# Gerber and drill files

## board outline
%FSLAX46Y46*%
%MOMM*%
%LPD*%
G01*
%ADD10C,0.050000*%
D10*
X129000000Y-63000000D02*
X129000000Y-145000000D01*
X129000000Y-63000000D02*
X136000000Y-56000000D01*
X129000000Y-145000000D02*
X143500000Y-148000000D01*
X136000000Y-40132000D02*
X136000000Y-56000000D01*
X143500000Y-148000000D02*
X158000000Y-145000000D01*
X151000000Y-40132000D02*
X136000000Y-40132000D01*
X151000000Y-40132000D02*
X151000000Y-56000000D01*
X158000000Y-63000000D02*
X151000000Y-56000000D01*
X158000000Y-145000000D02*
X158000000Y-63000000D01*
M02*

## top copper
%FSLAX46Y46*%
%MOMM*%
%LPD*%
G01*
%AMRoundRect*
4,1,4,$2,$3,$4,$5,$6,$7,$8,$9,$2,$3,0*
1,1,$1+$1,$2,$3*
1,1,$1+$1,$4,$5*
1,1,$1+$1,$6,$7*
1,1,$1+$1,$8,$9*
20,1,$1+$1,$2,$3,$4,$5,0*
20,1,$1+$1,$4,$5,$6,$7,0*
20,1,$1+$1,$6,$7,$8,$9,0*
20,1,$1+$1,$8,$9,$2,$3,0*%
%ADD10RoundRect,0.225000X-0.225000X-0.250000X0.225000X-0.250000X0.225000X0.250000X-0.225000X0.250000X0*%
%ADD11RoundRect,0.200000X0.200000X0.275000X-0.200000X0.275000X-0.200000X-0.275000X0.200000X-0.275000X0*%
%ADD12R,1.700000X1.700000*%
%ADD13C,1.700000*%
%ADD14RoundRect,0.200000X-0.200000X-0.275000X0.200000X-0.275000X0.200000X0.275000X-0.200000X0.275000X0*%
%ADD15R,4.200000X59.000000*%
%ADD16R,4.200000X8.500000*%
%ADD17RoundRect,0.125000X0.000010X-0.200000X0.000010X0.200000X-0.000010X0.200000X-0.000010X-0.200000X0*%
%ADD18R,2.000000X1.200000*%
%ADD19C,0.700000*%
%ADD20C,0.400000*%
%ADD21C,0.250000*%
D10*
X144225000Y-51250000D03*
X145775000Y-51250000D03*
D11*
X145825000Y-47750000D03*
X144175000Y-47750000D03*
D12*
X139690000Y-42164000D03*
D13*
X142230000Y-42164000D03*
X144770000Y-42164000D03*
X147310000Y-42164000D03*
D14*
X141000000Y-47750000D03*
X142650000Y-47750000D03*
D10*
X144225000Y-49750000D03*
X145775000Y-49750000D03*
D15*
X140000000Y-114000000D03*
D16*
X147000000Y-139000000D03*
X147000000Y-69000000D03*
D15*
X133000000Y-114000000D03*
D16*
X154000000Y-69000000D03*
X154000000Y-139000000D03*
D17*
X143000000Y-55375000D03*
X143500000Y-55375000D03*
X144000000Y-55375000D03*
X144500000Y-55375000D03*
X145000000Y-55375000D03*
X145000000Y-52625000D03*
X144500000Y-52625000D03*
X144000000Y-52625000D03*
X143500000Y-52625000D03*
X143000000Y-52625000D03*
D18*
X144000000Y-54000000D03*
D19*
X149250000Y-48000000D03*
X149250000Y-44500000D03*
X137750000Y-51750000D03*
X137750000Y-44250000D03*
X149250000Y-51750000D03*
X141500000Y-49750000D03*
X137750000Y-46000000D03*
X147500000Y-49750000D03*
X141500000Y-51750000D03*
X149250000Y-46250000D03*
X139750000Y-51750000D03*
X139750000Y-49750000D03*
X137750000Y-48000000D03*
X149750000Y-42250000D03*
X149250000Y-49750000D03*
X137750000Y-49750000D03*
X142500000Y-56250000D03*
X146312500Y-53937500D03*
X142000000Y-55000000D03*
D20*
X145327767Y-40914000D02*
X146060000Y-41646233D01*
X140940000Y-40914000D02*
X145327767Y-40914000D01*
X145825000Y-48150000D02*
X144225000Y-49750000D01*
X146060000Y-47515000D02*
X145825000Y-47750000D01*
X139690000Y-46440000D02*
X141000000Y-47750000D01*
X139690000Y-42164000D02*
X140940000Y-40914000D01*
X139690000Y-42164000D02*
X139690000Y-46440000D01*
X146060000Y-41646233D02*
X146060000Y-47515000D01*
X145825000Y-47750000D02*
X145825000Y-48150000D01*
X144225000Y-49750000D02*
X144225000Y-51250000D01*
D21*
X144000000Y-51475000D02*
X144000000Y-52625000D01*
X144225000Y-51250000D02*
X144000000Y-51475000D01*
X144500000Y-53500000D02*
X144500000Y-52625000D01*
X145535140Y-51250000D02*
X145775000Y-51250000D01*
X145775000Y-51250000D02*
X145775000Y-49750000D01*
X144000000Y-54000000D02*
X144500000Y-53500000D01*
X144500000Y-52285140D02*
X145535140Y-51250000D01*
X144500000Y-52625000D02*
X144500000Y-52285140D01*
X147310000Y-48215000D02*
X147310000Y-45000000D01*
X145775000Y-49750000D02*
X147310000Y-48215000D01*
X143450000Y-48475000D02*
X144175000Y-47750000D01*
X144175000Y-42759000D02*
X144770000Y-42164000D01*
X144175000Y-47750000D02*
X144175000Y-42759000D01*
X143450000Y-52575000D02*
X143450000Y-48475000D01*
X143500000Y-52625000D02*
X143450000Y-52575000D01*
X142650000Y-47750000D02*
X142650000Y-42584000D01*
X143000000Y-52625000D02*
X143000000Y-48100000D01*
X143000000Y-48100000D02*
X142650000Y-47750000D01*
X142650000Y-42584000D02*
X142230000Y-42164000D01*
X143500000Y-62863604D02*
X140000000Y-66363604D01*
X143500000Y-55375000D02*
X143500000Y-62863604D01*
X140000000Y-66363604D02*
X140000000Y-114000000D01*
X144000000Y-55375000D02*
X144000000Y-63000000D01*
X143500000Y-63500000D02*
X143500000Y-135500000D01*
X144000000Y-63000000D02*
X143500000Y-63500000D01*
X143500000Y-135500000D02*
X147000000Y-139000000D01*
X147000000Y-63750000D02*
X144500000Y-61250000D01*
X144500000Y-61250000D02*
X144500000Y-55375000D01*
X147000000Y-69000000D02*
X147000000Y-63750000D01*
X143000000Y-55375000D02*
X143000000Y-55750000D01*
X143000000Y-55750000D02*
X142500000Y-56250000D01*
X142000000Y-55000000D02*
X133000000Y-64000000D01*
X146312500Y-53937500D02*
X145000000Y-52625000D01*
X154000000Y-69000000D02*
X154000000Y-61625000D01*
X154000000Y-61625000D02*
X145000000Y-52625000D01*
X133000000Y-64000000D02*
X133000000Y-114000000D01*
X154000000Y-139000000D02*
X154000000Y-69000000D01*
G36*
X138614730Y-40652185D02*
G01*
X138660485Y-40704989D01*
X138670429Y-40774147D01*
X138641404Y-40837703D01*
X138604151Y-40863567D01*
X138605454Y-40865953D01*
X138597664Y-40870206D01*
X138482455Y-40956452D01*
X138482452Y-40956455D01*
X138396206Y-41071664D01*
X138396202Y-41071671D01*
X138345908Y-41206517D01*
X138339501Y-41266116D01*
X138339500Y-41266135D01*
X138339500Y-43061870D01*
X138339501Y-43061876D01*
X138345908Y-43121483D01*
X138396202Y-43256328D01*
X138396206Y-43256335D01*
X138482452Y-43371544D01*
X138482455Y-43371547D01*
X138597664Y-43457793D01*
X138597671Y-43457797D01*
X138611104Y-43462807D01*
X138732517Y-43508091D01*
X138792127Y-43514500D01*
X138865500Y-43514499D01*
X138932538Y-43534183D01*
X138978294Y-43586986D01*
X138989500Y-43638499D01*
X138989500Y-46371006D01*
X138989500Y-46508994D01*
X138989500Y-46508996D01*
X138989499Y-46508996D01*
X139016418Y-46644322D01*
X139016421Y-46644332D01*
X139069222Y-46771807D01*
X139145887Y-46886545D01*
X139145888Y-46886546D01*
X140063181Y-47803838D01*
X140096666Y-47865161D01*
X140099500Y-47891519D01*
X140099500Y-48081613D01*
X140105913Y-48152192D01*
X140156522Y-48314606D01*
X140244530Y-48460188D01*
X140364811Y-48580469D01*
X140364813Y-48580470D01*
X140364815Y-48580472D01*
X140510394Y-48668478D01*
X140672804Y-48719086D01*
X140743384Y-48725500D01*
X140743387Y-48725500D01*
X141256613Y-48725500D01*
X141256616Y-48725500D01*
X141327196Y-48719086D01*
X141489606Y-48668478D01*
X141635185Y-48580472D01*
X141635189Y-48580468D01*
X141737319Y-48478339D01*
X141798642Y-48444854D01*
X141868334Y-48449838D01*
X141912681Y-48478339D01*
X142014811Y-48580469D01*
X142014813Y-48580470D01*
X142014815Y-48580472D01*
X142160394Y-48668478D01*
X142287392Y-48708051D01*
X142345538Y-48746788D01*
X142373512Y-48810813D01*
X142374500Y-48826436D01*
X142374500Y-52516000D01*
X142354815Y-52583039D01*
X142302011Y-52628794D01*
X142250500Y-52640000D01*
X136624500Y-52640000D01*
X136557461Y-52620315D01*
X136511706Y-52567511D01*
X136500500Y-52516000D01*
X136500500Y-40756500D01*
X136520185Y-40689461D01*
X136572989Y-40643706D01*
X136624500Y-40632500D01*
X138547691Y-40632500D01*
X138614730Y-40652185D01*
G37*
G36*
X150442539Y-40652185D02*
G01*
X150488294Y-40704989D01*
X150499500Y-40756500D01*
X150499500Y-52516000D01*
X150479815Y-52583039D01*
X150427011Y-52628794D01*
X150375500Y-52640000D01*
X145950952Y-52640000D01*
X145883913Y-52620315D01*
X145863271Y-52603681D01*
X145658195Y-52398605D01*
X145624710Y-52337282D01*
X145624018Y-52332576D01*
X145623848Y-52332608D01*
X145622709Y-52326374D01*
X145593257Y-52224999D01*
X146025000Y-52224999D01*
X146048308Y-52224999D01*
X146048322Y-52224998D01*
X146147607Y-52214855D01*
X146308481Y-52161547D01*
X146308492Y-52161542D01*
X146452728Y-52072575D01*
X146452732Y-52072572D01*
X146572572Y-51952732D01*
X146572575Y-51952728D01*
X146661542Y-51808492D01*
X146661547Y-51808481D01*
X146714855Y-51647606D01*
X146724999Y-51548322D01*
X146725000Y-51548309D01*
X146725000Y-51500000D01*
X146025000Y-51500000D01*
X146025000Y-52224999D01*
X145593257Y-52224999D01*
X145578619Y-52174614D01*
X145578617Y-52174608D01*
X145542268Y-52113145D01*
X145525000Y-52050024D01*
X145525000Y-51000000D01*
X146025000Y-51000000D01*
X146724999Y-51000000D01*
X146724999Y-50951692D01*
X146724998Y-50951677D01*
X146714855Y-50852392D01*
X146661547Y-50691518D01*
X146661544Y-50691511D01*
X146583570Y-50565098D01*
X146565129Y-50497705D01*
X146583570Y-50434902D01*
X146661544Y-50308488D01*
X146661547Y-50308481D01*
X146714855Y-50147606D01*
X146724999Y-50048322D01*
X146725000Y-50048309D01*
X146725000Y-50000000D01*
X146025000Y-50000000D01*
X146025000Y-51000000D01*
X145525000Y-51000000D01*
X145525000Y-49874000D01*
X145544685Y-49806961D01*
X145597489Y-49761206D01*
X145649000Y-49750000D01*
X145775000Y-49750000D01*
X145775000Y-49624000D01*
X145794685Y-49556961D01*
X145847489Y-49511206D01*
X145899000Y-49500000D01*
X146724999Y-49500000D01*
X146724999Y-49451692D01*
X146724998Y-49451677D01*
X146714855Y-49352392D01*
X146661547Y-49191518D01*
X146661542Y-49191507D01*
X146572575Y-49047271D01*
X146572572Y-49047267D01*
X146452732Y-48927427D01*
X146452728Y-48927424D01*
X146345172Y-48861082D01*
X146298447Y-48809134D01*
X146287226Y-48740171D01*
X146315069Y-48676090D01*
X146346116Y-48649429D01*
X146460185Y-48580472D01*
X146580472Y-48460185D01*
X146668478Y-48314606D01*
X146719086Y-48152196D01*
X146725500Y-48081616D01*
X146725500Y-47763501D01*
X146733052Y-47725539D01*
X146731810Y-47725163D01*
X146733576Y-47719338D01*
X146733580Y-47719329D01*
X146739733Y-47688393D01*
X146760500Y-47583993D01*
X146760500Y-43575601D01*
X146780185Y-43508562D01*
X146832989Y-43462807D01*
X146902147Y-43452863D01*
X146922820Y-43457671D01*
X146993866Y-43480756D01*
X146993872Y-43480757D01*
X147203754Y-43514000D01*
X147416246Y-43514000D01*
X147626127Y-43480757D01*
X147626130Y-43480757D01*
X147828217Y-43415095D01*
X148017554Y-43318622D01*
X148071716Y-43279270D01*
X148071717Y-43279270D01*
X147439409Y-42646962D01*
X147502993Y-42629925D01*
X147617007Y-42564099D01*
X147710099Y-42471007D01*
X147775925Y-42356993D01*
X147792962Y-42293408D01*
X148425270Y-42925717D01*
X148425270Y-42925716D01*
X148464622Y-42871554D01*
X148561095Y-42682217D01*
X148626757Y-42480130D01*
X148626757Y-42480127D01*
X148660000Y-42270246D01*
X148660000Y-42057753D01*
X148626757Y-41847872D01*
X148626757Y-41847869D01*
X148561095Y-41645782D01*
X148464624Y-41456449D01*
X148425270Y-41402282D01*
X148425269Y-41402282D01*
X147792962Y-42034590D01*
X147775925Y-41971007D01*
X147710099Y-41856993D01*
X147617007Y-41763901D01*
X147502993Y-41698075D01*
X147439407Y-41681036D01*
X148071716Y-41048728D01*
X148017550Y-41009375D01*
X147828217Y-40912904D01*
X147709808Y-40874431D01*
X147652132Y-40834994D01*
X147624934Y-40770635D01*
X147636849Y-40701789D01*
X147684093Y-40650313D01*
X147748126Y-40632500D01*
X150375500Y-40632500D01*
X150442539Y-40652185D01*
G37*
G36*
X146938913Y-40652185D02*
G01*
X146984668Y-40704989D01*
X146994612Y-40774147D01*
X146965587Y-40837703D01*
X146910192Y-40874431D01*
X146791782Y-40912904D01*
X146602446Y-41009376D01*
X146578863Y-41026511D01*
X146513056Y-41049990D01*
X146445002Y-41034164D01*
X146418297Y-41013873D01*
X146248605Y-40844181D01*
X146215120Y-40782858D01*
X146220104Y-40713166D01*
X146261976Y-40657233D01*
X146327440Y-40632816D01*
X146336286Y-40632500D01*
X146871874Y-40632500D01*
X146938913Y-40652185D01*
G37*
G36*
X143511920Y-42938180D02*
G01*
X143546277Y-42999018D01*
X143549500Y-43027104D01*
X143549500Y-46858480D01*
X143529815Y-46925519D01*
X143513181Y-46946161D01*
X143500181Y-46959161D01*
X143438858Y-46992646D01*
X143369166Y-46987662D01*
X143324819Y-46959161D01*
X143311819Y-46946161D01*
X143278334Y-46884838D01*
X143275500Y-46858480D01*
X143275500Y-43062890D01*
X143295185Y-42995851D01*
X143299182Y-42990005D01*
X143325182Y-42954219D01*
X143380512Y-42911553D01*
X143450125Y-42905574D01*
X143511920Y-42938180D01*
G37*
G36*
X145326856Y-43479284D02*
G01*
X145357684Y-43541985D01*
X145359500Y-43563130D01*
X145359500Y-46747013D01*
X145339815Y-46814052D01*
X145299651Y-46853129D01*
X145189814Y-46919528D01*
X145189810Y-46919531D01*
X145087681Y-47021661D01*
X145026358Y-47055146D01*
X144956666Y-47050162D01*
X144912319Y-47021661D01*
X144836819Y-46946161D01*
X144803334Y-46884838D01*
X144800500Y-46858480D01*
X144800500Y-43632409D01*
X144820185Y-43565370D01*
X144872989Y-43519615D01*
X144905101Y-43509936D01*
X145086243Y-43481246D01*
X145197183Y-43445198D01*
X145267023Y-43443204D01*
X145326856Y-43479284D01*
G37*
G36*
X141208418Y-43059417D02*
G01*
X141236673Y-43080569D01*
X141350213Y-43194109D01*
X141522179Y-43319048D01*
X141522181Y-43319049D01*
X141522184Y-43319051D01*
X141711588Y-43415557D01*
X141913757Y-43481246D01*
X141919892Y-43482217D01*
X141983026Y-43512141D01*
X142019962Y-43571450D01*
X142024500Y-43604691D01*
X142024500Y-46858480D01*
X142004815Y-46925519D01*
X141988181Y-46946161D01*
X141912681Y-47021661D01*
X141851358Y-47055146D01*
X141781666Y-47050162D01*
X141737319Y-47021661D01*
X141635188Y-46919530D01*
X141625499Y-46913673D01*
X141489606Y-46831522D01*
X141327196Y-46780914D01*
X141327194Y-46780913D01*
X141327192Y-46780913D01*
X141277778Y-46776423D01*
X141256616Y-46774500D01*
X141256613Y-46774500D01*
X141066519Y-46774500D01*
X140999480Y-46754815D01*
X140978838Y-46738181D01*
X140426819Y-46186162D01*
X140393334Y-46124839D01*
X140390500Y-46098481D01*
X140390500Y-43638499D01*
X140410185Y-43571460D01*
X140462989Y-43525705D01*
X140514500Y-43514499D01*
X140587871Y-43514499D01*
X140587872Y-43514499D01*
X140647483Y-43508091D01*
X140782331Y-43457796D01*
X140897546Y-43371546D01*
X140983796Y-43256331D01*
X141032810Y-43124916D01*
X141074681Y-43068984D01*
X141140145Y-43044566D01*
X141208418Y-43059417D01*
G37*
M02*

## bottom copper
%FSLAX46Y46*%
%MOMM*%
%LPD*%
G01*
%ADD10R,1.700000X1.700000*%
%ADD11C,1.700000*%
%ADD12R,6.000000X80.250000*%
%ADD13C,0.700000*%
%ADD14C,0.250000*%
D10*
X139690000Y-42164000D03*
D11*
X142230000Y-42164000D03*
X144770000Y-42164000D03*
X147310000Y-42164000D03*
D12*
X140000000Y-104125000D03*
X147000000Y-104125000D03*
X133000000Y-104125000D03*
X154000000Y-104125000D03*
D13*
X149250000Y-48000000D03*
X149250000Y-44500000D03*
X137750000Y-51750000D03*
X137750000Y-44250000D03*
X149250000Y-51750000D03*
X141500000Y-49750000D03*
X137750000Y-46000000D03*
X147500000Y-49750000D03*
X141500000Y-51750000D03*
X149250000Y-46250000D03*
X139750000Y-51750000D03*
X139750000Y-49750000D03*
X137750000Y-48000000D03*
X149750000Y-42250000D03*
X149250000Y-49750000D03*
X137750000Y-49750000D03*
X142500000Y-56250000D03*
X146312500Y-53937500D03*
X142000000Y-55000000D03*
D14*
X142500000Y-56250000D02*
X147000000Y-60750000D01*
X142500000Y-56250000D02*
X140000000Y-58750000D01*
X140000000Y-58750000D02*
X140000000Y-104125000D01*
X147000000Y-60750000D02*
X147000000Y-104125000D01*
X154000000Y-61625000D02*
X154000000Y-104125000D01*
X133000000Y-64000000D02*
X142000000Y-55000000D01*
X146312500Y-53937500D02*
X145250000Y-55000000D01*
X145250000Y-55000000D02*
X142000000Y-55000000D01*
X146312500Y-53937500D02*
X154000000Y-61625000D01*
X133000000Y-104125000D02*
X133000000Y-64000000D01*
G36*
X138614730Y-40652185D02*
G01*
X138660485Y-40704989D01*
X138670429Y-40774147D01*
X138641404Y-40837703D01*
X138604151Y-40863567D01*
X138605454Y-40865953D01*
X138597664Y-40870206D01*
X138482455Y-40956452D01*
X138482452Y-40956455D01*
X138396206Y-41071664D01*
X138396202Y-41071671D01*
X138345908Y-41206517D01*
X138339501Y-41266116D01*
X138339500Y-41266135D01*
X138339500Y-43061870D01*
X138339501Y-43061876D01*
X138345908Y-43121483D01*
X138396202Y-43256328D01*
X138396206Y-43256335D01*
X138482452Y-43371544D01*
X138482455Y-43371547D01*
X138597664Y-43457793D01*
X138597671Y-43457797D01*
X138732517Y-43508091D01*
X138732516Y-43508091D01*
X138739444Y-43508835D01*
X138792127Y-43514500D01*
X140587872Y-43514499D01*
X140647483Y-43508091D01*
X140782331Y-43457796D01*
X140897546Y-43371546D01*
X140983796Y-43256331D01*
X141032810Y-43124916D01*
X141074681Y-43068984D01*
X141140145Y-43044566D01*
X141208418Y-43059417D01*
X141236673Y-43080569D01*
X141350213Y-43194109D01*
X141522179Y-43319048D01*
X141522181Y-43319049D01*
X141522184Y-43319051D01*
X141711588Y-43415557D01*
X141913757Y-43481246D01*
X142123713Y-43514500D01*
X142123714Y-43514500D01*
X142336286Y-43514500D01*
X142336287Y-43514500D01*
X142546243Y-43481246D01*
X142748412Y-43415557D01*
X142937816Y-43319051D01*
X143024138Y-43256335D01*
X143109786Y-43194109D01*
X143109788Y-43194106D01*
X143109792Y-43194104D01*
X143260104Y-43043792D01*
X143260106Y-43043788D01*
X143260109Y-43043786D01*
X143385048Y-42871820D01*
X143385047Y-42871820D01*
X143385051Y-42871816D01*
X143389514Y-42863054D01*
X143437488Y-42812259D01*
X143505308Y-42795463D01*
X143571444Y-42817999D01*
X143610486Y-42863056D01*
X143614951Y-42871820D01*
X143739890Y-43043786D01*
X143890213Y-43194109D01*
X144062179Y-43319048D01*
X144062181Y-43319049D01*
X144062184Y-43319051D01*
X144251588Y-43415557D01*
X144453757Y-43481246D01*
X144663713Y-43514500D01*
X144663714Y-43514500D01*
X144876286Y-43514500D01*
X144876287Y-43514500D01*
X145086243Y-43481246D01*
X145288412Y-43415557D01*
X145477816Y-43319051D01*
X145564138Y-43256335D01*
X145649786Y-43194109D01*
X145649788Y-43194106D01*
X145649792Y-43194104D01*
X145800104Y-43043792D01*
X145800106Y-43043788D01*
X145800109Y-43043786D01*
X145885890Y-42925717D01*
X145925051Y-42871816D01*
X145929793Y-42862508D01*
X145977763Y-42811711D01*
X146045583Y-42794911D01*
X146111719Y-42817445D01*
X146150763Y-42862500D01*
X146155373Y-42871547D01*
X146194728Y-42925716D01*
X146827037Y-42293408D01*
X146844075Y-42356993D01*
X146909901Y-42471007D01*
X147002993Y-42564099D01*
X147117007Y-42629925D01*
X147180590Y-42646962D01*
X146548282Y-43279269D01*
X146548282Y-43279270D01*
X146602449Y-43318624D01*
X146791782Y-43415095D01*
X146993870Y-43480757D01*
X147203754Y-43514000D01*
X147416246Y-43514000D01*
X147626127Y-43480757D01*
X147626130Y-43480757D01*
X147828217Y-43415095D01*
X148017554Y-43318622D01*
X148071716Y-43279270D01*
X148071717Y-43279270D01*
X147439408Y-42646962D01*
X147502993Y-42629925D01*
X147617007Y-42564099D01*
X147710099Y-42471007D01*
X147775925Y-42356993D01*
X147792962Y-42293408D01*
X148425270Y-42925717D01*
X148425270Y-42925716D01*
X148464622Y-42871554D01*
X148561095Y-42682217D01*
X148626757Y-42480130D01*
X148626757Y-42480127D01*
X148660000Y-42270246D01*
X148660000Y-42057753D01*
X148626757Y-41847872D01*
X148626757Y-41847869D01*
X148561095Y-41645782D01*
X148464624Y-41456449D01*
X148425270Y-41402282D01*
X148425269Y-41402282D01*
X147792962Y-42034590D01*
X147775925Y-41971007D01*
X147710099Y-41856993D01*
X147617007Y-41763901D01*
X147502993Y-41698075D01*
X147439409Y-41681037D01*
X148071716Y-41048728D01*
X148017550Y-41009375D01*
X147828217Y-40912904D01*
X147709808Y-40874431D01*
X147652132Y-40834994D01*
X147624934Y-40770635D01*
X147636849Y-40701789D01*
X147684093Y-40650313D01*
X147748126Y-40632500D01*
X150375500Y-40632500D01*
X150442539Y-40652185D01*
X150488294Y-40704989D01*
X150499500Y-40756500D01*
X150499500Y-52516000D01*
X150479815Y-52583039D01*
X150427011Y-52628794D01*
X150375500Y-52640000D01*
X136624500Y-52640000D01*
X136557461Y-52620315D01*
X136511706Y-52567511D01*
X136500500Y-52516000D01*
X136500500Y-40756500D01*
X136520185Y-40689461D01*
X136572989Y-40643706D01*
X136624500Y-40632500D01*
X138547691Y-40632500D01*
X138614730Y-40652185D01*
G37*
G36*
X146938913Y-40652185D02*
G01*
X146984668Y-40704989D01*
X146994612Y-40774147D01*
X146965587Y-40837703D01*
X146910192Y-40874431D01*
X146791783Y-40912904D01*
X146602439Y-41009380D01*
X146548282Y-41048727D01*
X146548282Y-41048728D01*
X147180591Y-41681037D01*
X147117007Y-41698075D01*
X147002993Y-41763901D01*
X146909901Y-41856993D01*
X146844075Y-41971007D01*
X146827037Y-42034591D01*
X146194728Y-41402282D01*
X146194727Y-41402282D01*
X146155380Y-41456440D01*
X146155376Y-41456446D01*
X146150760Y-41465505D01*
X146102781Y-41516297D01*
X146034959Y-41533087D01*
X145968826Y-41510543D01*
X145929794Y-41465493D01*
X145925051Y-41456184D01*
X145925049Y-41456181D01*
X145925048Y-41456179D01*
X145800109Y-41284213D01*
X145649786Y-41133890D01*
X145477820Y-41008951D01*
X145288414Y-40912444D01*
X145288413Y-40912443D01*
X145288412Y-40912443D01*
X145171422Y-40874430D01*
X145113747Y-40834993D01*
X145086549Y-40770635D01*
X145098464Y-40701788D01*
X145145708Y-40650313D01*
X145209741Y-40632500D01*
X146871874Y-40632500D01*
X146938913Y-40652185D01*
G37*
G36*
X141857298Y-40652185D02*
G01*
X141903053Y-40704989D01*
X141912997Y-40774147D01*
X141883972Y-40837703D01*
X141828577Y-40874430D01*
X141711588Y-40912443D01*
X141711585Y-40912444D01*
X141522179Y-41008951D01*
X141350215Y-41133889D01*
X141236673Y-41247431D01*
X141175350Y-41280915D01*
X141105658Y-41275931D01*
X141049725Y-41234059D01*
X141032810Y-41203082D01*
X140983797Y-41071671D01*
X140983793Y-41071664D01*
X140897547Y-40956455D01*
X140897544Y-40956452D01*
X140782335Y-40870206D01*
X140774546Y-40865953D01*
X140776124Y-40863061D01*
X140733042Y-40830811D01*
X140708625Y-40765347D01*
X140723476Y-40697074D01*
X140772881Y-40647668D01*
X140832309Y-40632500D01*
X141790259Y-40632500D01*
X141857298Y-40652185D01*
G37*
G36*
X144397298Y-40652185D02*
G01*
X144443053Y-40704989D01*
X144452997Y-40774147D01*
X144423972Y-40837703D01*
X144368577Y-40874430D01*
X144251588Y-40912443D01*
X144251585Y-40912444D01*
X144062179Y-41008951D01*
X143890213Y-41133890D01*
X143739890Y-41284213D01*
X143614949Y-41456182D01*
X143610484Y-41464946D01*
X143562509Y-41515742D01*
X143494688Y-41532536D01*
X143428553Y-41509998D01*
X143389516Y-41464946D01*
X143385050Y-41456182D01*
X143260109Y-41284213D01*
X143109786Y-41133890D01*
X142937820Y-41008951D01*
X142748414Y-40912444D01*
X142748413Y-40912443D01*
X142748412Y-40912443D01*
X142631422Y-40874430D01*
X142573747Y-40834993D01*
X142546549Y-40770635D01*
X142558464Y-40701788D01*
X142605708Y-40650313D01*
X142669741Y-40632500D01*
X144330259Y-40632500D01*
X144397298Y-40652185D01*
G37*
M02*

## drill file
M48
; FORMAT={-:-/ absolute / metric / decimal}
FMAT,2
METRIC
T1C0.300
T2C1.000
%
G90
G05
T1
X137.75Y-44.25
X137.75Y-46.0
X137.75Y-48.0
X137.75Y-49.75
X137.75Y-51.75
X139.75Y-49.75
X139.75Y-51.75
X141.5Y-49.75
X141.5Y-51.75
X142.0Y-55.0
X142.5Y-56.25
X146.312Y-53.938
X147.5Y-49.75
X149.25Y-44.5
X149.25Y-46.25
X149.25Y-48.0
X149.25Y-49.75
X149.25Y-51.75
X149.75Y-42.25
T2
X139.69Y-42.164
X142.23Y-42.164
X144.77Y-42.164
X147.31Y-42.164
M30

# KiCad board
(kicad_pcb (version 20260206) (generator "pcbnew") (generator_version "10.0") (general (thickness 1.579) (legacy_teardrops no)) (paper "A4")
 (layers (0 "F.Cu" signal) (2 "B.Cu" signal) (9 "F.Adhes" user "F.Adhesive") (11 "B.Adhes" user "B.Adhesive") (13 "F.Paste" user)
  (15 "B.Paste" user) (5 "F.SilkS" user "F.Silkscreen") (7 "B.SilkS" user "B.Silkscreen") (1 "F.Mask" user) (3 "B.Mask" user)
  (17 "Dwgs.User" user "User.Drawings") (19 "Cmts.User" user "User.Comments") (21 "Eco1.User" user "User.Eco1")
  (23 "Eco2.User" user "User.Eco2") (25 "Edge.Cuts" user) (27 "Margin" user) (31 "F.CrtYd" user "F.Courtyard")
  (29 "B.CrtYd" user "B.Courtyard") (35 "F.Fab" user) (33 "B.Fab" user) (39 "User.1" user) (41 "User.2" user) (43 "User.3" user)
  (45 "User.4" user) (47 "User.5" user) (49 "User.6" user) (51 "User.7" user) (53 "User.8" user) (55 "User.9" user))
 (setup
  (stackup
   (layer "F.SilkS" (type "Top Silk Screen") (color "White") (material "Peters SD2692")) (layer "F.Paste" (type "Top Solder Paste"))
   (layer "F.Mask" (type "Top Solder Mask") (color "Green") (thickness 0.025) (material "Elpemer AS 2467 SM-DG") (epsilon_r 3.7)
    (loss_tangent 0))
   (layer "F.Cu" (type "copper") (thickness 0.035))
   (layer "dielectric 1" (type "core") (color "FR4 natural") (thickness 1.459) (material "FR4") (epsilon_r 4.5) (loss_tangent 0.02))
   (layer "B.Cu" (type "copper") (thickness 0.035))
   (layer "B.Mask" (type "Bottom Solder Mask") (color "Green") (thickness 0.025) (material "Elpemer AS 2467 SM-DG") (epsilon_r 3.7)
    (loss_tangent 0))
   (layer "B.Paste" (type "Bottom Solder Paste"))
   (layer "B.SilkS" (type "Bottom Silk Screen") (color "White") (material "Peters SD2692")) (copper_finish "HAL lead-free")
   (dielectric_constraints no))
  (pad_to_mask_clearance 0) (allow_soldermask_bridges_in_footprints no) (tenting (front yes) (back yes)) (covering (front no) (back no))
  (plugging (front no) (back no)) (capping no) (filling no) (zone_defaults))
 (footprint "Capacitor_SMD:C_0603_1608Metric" (layer "F.Cu") (at 145 51.25)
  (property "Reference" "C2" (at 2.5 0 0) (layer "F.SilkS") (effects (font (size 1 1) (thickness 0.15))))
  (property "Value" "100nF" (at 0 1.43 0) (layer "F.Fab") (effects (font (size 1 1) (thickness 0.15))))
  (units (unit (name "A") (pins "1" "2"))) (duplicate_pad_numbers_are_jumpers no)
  (pad "1" smd roundrect (at -0.775 0) (size 0.9 0.95) (layers "F.Cu" "F.Mask" "F.Paste") (roundrect_rratio 0.25) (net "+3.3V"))
  (pad "2" smd roundrect (at 0.775 0) (size 0.9 0.95) (layers "F.Cu" "F.Mask" "F.Paste") (roundrect_rratio 0.25) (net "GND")))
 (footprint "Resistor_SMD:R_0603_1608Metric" (layer "F.Cu") (at 145 47.75 180)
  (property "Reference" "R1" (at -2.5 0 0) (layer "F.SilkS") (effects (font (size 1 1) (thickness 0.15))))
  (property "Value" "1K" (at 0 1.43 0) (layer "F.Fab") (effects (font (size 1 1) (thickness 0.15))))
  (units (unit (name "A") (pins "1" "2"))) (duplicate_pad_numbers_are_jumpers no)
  (pad "1" smd roundrect (at -0.825 0 180) (size 0.8 0.95) (layers "F.Cu" "F.Mask" "F.Paste") (roundrect_rratio 0.25) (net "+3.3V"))
  (pad "2" smd roundrect (at 0.825 0 180) (size 0.8 0.95) (layers "F.Cu" "F.Mask" "F.Paste") (roundrect_rratio 0.25) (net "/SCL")))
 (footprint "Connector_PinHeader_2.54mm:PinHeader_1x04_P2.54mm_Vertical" (layer "F.Cu") (at 139.69 42.164 90)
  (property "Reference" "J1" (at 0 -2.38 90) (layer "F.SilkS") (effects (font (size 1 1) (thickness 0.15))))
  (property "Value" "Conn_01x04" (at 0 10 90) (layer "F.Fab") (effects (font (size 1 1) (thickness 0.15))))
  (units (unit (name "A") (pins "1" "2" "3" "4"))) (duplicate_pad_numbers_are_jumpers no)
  (pad "1" thru_hole rect (at 0 0 90) (size 1.7 1.7) (drill 1) (layers "*.Cu" "*.Mask") (remove_unused_layers no) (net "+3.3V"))
  (pad "2" thru_hole circle (at 0 2.54 90) (size 1.7 1.7) (drill 1) (layers "*.Cu" "*.Mask") (remove_unused_layers no) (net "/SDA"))
  (pad "3" thru_hole circle (at 0 5.08 90) (size 1.7 1.7) (drill 1) (layers "*.Cu" "*.Mask") (remove_unused_layers no) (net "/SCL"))
  (pad "4" thru_hole circle (at 0 7.62 90) (size 1.7 1.7) (drill 1) (layers "*.Cu" "*.Mask") (remove_unused_layers no) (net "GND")))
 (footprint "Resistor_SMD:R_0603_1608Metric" (layer "F.Cu") (at 141.825 47.75)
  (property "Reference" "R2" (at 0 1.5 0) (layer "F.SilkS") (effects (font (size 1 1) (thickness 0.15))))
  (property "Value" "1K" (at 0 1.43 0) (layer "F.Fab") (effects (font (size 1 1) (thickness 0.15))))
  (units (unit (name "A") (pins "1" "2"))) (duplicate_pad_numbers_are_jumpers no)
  (pad "1" smd roundrect (at -0.825 0) (size 0.8 0.95) (layers "F.Cu" "F.Mask" "F.Paste") (roundrect_rratio 0.25) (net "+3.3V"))
  (pad "2" smd roundrect (at 0.825 0) (size 0.8 0.95) (layers "F.Cu" "F.Mask" "F.Paste") (roundrect_rratio 0.25) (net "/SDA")))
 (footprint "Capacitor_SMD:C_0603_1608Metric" (layer "F.Cu") (at 145 49.75)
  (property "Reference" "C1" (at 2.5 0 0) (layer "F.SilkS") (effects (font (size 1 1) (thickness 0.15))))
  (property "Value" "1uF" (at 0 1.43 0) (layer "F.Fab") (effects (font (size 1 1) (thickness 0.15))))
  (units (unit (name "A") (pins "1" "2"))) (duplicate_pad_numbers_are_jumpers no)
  (pad "1" smd roundrect (at -0.775 0) (size 0.9 0.95) (layers "F.Cu" "F.Mask" "F.Paste") (roundrect_rratio 0.25) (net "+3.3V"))
  (pad "2" smd roundrect (at 0.775 0) (size 0.9 0.95) (layers "F.Cu" "F.Mask" "F.Paste") (roundrect_rratio 0.25) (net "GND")))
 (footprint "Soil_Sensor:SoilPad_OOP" (layer "F.Cu") (at 143.5 103)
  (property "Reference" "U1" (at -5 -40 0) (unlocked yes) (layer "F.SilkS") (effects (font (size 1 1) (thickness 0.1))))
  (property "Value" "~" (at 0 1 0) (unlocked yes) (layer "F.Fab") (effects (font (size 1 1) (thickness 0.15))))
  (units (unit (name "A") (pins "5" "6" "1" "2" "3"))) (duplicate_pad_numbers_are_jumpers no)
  (pad "1" smd rect (at -3.5 11) (size 4.2 59) (layers "F.Cu") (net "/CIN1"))
  (pad "2" smd rect (at 3.5 36) (size 4.2 8.5) (layers "F.Cu") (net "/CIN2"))
  (pad "3" smd rect (at 3.5 -34) (size 4.2 8.5) (layers "F.Cu") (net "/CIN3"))
  (pad "5" smd rect (at -3.5 1.125) (size 6 80.25) (layers "B.Cu") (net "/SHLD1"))
  (pad "5" smd rect (at 3.5 1.125) (size 6 80.25) (layers "B.Cu") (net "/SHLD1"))
  (pad "6" smd rect (at -10.5 1.125) (size 6 80.25) (layers "B.Cu") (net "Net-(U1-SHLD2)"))
  (pad "6" smd rect (at -10.5 11) (size 4.2 59) (layers "F.Cu") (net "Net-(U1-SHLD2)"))
  (pad "6" smd rect (at 10.5 -34) (size 4.2 8.5) (layers "F.Cu") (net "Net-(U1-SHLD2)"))
  (pad "6" smd rect (at 10.5 1.125) (size 6 80.25) (layers "B.Cu") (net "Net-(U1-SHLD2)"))
  (pad "6" smd rect (at 10.5 36) (size 4.2 8.5) (layers "F.Cu") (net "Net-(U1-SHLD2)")))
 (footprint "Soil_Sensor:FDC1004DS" (layer "F.Cu") (at 144 54 90)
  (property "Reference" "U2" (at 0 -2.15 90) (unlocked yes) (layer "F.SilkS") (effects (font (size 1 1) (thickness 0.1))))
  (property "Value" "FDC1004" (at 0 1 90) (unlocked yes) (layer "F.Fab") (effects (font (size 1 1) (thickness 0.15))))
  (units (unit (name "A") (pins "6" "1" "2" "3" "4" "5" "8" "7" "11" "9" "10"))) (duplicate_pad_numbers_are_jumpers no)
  (pad "1" smd roundrect (at -1.375 -1 90) (size 0.65 0.25) (layers "F.Cu" "F.Mask" "F.Paste") (roundrect_rratio 0.5) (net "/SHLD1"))
  (pad "2" smd roundrect (at -1.375 -0.5 90) (size 0.65 0.25) (layers "F.Cu" "F.Mask" "F.Paste") (roundrect_rratio 0.5) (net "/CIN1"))
  (pad "3" smd roundrect (at -1.375 0 90) (size 0.65 0.25) (layers "F.Cu" "F.Mask" "F.Paste") (roundrect_rratio 0.5) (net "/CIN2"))
  (pad "4" smd roundrect (at -1.375 0.5 90) (size 0.65 0.25) (layers "F.Cu" "F.Mask" "F.Paste") (roundrect_rratio 0.5) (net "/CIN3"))
  (pad "5" smd roundrect (at -1.375 1 90) (size 0.65 0.25) (layers "F.Cu" "F.Mask" "F.Paste") (roundrect_rratio 0.5)
   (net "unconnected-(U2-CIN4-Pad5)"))
  (pad "6" smd roundrect (at 1.375 1 90) (size 0.65 0.25) (layers "F.Cu" "F.Mask" "F.Paste") (roundrect_rratio 0.5) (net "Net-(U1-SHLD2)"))
  (pad "7" smd roundrect (at 1.375 0.5 90) (size 0.65 0.25) (layers "F.Cu" "F.Mask" "F.Paste") (roundrect_rratio 0.5) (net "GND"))
  (pad "8" smd roundrect (at 1.375 0 90) (size 0.65 0.25) (layers "F.Cu" "F.Mask" "F.Paste") (roundrect_rratio 0.5) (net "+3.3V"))
  (pad "9" smd roundrect (at 1.375 -0.5 90) (size 0.65 0.25) (layers "F.Cu" "F.Mask" "F.Paste") (roundrect_rratio 0.5) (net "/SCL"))
  (pad "10" smd roundrect (at 1.375 -1 90) (size 0.65 0.25) (layers "F.Cu" "F.Mask" "F.Paste") (roundrect_rratio 0.5) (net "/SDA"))
  (pad "11" smd rect (at 0 0 90) (size 1.2 2) (layers "F.Cu" "F.Mask" "F.Paste") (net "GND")))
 (gr_line (start 129 63) (end 129 145) (stroke (width 0.05) (type default)) (layer "Edge.Cuts"))
 (gr_line (start 129 63) (end 136 56) (stroke (width 0.05) (type default)) (layer "Edge.Cuts"))
 (gr_line (start 129 145) (end 143.5 148) (stroke (width 0.05) (type default)) (layer "Edge.Cuts"))
 (gr_line (start 136 40.132) (end 136 56) (stroke (width 0.05) (type default)) (layer "Edge.Cuts"))
 (gr_line (start 143.5 148) (end 158 145) (stroke (width 0.05) (type default)) (layer "Edge.Cuts"))
 (gr_line (start 151 40.132) (end 136 40.132) (stroke (width 0.05) (type default)) (layer "Edge.Cuts"))
 (gr_line (start 151 40.132) (end 151 56) (stroke (width 0.05) (type default)) (layer "Edge.Cuts"))
 (gr_line (start 158 63) (end 151 56) (stroke (width 0.05) (type default)) (layer "Edge.Cuts"))
 (gr_line (start 158 145) (end 158 63) (stroke (width 0.05) (type default)) (layer "Edge.Cuts"))
 (segment (start 145.327767 40.914) (end 146.06 41.646233) (width 0.4) (layer "F.Cu") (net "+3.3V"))
 (segment (start 140.94 40.914) (end 145.327767 40.914) (width 0.4) (layer "F.Cu") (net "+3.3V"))
 (segment (start 145.825 48.15) (end 144.225 49.75) (width 0.4) (layer "F.Cu") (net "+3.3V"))
 (segment (start 146.06 47.515) (end 145.825 47.75) (width 0.4) (layer "F.Cu") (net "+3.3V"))
 (segment (start 139.69 46.44) (end 141 47.75) (width 0.4) (layer "F.Cu") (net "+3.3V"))
 (segment (start 139.69 42.164) (end 140.94 40.914) (width 0.4) (layer "F.Cu") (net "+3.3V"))
 (segment (start 139.69 42.164) (end 139.69 46.44) (width 0.4) (layer "F.Cu") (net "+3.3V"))
 (segment (start 146.06 41.646233) (end 146.06 47.515) (width 0.4) (layer "F.Cu") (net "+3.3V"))
 (segment (start 145.825 47.75) (end 145.825 48.15) (width 0.4) (layer "F.Cu") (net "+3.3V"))
 (segment (start 144.225 49.75) (end 144.225 51.25) (width 0.4) (layer "F.Cu") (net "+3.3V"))
 (segment (start 144 51.475) (end 144 52.625) (width 0.25) (layer "F.Cu") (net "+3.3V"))
 (segment (start 144.225 51.25) (end 144 51.475) (width 0.25) (layer "F.Cu") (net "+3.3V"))
 (segment (start 144.5 53.5) (end 144.5 52.625) (width 0.25) (layer "F.Cu") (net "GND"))
 (segment (start 145.53514 51.25) (end 145.775 51.25) (width 0.25) (layer "F.Cu") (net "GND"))
 (segment (start 145.775 51.25) (end 145.775 49.75) (width 0.25) (layer "F.Cu") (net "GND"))
 (segment (start 144 54) (end 144.5 53.5) (width 0.25) (layer "F.Cu") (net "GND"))
 (segment (start 144.5 52.28514) (end 145.53514 51.25) (width 0.25) (layer "F.Cu") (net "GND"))
 (segment (start 144.5 52.625) (end 144.5 52.28514) (width 0.25) (layer "F.Cu") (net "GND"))
 (segment (start 147.31 48.215) (end 147.31 45) (width 0.25) (layer "F.Cu") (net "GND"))
 (segment (start 145.775 49.75) (end 147.31 48.215) (width 0.25) (layer "F.Cu") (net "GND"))
 (via (at 149.25 48) (size 0.7) (drill 0.3) (layers "F.Cu" "B.Cu") (free yes) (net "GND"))
 (via (at 149.25 44.5) (size 0.7) (drill 0.3) (layers "F.Cu" "B.Cu") (free yes) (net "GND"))
 (via (at 137.75 51.75) (size 0.7) (drill 0.3) (layers "F.Cu" "B.Cu") (free yes) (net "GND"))
 (via (at 137.75 44.25) (size 0.7) (drill 0.3) (layers "F.Cu" "B.Cu") (free yes) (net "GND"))
 (via (at 149.25 51.75) (size 0.7) (drill 0.3) (layers "F.Cu" "B.Cu") (free yes) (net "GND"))
 (via (at 141.5 49.75) (size 0.7) (drill 0.3) (layers "F.Cu" "B.Cu") (free yes) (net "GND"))
 (via (at 137.75 46) (size 0.7) (drill 0.3) (layers "F.Cu" "B.Cu") (free yes) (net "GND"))
 (via (at 147.5 49.75) (size 0.7) (drill 0.3) (layers "F.Cu" "B.Cu") (free yes) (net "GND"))
 (via (at 141.5 51.75) (size 0.7) (drill 0.3) (layers "F.Cu" "B.Cu") (free yes) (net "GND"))
 (via (at 149.25 46.25) (size 0.7) (drill 0.3) (layers "F.Cu" "B.Cu") (free yes) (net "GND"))
 (via (at 139.75 51.75) (size 0.7) (drill 0.3) (layers "F.Cu" "B.Cu") (free yes) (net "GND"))
 (via (at 139.75 49.75) (size 0.7) (drill 0.3) (layers "F.Cu" "B.Cu") (free yes) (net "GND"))
 (via (at 137.75 48) (size 0.7) (drill 0.3) (layers "F.Cu" "B.Cu") (free yes) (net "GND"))
 (via (at 149.75 42.25) (size 0.7) (drill 0.3) (layers "F.Cu" "B.Cu") (free yes) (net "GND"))
 (via (at 149.25 49.75) (size 0.7) (drill 0.3) (layers "F.Cu" "B.Cu") (free yes) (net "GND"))
 (via (at 137.75 49.75) (size 0.7) (drill 0.3) (layers "F.Cu" "B.Cu") (free yes) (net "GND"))
 (segment (start 143.45 48.475) (end 144.175 47.75) (width 0.25) (layer "F.Cu") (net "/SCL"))
 (segment (start 144.175 42.759) (end 144.77 42.164) (width 0.25) (layer "F.Cu") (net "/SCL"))
 (segment (start 144.175 47.75) (end 144.175 42.759) (width 0.25) (layer "F.Cu") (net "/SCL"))
 (segment (start 143.45 52.575) (end 143.45 48.475) (width 0.25) (layer "F.Cu") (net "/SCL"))
 (segment (start 143.5 52.625) (end 143.45 52.575) (width 0.25) (layer "F.Cu") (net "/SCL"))
 (segment (start 142.65 47.75) (end 142.65 42.584) (width 0.25) (layer "F.Cu") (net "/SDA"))
 (segment (start 143 52.625) (end 143 48.1) (width 0.25) (layer "F.Cu") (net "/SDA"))
 (segment (start 143 48.1) (end 142.65 47.75) (width 0.25) (layer "F.Cu") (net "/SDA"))
 (segment (start 142.65 42.584) (end 142.23 42.164) (width 0.25) (layer "F.Cu") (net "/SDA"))
 (segment (start 143.5 62.863604) (end 140 66.363604) (width 0.25) (layer "F.Cu") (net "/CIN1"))
 (segment (start 143.5 55.375) (end 143.5 62.863604) (width 0.25) (layer "F.Cu") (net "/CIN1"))
 (segment (start 140 66.363604) (end 140 114) (width 0.25) (layer "F.Cu") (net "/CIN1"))
 (segment (start 144 55.375) (end 144 63) (width 0.25) (layer "F.Cu") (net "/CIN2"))
 (segment (start 143.5 63.5) (end 143.5 135.5) (width 0.25) (layer "F.Cu") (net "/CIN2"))
 (segment (start 144 63) (end 143.5 63.5) (width 0.25) (layer "F.Cu") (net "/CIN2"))
 (segment (start 143.5 135.5) (end 147 139) (width 0.25) (layer "F.Cu") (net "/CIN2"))
 (segment (start 147 63.75) (end 144.5 61.25) (width 0.25) (layer "F.Cu") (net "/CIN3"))
 (segment (start 144.5 61.25) (end 144.5 55.375) (width 0.25) (layer "F.Cu") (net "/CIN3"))
 (segment (start 147 69) (end 147 63.75) (width 0.25) (layer "F.Cu") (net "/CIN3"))
 (segment (start 143 55.375) (end 143 55.75) (width 0.25) (layer "F.Cu") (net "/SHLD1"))
 (segment (start 143 55.75) (end 142.5 56.25) (width 0.25) (layer "F.Cu") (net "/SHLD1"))
 (via (at 142.5 56.25) (size 0.7) (drill 0.3) (layers "F.Cu" "B.Cu") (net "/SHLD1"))
 (segment (start 142.5 56.25) (end 147 60.75) (width 0.25) (layer "B.Cu") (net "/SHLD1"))
 (segment (start 142.5 56.25) (end 140 58.75) (width 0.25) (layer "B.Cu") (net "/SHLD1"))
 (segment (start 140 58.75) (end 140 104.125) (width 0.25) (layer "B.Cu") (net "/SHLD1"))
 (segment (start 147 60.75) (end 147 104.125) (width 0.25) (layer "B.Cu") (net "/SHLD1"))
 (segment (start 142 55) (end 133 64) (width 0.25) (layer "F.Cu") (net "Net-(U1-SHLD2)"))
 (segment (start 146.3125 53.9375) (end 145 52.625) (width 0.25) (layer "F.Cu") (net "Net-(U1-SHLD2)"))
 (segment (start 154 69) (end 154 61.625) (width 0.25) (layer "F.Cu") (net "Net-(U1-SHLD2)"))
 (segment (start 154 61.625) (end 145 52.625) (width 0.25) (layer "F.Cu") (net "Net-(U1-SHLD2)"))
 (segment (start 133 64) (end 133 114) (width 0.25) (layer "F.Cu") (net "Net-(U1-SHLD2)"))
 (segment (start 154 139) (end 154 69) (width 0.25) (layer "F.Cu") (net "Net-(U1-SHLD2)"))
 (via (at 146.3125 53.9375) (size 0.7) (drill 0.3) (layers "F.Cu" "B.Cu") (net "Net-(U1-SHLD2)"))
 (via (at 142 55) (size 0.7) (drill 0.3) (layers "F.Cu" "B.Cu") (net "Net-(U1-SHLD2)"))
 (segment (start 154 61.625) (end 154 104.125) (width 0.25) (layer "B.Cu") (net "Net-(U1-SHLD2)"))
 (segment (start 133 64) (end 142 55) (width 0.25) (layer "B.Cu") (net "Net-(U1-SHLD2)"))
 (segment (start 146.3125 53.9375) (end 145.25 55) (width 0.25) (layer "B.Cu") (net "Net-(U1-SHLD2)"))
 (segment (start 145.25 55) (end 142 55) (width 0.25) (layer "B.Cu") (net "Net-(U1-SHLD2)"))
 (segment (start 146.3125 53.9375) (end 154 61.625) (width 0.25) (layer "B.Cu") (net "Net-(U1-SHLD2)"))
 (segment (start 133 104.125) (end 133 64) (width 0.25) (layer "B.Cu") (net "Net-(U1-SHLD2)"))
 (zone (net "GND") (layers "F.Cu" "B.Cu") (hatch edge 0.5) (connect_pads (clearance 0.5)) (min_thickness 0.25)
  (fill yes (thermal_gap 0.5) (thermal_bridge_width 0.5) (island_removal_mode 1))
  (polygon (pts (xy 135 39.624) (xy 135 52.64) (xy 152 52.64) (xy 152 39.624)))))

